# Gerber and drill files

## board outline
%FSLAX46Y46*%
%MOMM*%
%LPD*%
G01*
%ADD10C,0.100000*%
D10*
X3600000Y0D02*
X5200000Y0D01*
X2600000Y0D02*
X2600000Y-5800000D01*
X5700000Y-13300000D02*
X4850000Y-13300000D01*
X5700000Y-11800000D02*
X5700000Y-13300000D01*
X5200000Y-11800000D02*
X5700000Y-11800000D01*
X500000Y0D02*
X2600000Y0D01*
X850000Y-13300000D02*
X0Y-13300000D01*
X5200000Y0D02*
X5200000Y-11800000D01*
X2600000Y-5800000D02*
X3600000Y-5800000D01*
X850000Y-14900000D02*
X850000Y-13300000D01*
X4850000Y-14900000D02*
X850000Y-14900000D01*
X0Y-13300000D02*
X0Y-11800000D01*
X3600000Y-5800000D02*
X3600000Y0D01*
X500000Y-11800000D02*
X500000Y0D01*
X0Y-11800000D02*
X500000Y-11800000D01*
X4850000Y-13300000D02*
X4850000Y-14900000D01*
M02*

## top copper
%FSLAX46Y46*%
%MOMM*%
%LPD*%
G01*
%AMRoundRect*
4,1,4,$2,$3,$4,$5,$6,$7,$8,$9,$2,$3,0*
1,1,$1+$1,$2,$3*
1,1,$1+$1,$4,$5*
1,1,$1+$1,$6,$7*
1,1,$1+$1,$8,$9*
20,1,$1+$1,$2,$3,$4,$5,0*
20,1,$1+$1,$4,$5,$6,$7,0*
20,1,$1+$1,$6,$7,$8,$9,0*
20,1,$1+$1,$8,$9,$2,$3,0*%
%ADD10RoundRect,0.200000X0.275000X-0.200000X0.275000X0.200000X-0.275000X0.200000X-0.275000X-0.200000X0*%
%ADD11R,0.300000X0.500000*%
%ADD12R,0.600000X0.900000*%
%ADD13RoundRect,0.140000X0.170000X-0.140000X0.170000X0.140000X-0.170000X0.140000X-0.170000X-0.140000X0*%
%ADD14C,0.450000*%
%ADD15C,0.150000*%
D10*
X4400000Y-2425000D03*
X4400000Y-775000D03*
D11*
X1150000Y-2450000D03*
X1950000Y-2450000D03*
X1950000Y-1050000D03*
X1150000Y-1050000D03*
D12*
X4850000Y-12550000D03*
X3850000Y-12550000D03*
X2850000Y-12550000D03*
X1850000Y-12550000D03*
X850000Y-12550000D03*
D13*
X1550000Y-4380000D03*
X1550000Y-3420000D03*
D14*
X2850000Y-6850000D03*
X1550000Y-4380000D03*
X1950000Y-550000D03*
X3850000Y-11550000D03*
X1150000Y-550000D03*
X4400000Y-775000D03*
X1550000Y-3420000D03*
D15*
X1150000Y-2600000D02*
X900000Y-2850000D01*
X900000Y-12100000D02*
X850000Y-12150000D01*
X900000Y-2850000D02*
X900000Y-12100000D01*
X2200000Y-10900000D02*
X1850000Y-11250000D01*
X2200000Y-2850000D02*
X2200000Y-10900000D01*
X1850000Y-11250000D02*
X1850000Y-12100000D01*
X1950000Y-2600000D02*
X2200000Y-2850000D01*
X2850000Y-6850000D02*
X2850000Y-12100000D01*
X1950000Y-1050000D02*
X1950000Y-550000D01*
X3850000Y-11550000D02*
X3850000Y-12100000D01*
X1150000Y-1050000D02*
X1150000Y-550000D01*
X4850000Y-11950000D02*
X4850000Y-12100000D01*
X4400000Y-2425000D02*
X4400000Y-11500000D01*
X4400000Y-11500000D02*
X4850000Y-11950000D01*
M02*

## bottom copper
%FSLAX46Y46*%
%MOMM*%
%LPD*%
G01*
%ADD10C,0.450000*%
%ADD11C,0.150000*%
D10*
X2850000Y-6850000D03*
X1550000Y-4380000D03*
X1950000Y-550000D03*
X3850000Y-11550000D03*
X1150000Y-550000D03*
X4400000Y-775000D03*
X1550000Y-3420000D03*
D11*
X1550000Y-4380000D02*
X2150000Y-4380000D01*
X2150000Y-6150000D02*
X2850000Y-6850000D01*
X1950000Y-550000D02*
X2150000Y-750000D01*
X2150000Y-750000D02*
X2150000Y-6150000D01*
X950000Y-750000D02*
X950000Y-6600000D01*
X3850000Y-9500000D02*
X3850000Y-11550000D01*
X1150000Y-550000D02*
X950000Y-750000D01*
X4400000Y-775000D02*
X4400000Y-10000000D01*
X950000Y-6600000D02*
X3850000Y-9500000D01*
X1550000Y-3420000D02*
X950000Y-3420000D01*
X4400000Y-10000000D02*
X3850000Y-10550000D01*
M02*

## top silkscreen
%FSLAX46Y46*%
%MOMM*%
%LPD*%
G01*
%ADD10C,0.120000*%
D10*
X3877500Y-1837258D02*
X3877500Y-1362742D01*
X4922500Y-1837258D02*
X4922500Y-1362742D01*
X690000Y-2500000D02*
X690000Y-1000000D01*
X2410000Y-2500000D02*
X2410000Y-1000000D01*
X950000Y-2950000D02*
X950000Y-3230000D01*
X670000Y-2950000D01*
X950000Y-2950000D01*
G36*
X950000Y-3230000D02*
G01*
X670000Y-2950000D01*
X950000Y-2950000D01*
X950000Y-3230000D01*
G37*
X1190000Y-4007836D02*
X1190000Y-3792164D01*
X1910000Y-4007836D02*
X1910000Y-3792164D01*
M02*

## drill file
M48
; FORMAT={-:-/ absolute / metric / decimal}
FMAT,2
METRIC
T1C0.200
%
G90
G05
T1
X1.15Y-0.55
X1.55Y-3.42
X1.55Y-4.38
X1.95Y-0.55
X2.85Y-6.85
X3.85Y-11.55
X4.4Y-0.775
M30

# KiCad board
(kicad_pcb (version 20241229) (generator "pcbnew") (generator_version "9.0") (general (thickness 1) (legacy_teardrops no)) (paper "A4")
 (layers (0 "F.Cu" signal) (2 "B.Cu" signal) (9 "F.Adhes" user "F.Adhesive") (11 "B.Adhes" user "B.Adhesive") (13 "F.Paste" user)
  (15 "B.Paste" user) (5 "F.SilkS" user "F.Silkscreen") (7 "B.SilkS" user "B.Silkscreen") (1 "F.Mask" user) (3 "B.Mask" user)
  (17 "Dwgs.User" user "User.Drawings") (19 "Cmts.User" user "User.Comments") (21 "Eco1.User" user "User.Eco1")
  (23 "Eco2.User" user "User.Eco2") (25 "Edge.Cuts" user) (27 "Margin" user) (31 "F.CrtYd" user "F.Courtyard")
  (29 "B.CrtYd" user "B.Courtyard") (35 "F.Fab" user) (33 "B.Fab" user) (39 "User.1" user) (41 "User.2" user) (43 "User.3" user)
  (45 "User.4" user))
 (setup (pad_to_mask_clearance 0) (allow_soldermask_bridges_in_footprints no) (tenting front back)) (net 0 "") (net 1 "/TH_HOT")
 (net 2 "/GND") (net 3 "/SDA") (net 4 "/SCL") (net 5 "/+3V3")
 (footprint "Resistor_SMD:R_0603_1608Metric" (layer "F.Cu") (at 4.4 1.6 90)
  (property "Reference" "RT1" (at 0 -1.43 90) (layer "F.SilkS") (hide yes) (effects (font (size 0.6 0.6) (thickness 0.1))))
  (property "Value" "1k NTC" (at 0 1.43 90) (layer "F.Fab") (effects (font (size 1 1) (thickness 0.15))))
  (fp_line (start -0.237258 -0.5225) (end 0.237258 -0.5225) (stroke (width 0.12) (type solid)) (layer "F.SilkS"))
  (fp_line (start -0.237258 0.5225) (end 0.237258 0.5225) (stroke (width 0.12) (type solid)) (layer "F.SilkS"))
  (pad "1" smd roundrect (at -0.825 0 90) (size 0.8 0.95) (layers "F.Cu" "F.Mask" "F.Paste") (roundrect_rratio 0.25) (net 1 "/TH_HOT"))
  (pad "2" smd roundrect (at 0.825 0 90) (size 0.8 0.95) (layers "F.Cu" "F.Mask" "F.Paste") (roundrect_rratio 0.25) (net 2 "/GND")))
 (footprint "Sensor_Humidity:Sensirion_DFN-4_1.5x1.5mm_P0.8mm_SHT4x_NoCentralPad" (layer "F.Cu") (at 1.55 1.75 90)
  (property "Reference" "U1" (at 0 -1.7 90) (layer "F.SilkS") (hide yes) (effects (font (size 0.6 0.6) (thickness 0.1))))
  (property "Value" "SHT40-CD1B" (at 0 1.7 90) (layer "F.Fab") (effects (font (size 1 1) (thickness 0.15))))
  (fp_line (start -0.75 -0.86) (end 0.75 -0.86) (stroke (width 0.12) (type solid)) (layer "F.SilkS"))
  (fp_line (start -0.75 0.86) (end 0.75 0.86) (stroke (width 0.12) (type solid)) (layer "F.SilkS"))
  (fp_poly
   (pts (xy -1.2 -0.6) (xy -1.48 -0.6) (xy -1.2 -0.88) (xy -1.2 -0.6)) (stroke (width 0.12) (type solid)) (fill yes) (layer "F.SilkS"))
  (pad "1" smd rect (at -0.7 -0.4 90) (size 0.5 0.3) (layers "F.Cu" "F.Mask" "F.Paste") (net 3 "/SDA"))
  (pad "2" smd rect (at -0.7 0.4 90) (size 0.5 0.3) (layers "F.Cu" "F.Mask" "F.Paste") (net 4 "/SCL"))
  (pad "3" smd rect (at 0.7 0.4 90) (size 0.5 0.3) (layers "F.Cu" "F.Mask" "F.Paste") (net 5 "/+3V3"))
  (pad "4" smd rect (at 0.7 -0.4 90) (size 0.5 0.3) (layers "F.Cu" "F.Mask" "F.Paste") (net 2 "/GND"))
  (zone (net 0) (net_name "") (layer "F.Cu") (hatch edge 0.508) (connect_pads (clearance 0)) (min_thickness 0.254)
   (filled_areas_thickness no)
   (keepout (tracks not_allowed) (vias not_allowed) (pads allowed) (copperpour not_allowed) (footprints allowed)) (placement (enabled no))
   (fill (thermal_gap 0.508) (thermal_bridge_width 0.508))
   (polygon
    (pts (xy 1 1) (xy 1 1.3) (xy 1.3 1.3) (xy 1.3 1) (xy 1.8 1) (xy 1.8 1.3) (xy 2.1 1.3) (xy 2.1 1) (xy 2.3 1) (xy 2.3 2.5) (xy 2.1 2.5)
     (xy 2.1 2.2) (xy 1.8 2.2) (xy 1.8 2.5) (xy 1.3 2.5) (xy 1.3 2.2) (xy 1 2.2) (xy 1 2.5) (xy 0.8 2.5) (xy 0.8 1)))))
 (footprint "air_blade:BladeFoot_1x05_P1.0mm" (layer "F.Cu") (at 2.85 12.55)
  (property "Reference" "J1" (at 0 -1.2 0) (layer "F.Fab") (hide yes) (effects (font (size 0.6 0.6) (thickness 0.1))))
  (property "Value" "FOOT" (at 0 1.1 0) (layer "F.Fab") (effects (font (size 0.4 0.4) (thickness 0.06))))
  (pad "1" smd rect (at 2 0) (size 0.6 0.9) (layers "F.Cu" "F.Mask" "F.Paste") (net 1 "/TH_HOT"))
  (pad "2" smd rect (at 1 0) (size 0.6 0.9) (layers "F.Cu" "F.Mask" "F.Paste") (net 2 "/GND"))
  (pad "3" smd rect (at 0 0) (size 0.6 0.9) (layers "F.Cu" "F.Mask" "F.Paste") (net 5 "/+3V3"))
  (pad "4" smd rect (at -1 0) (size 0.6 0.9) (layers "F.Cu" "F.Mask" "F.Paste") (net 4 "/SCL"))
  (pad "5" smd rect (at -2 0) (size 0.6 0.9) (layers "F.Cu" "F.Mask" "F.Paste") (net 3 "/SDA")))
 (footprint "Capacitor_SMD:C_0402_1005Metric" (layer "F.Cu") (at 1.55 3.9 90)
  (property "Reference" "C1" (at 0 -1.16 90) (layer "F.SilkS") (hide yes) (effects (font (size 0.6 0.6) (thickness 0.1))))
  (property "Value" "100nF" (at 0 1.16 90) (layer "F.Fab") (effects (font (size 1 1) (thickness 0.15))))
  (fp_line (start -0.107836 -0.36) (end 0.107836 -0.36) (stroke (width 0.12) (type solid)) (layer "F.SilkS"))
  (fp_line (start -0.107836 0.36) (end 0.107836 0.36) (stroke (width 0.12) (type solid)) (layer "F.SilkS"))
  (pad "1" smd roundrect (at -0.48 0 90) (size 0.56 0.62) (layers "F.Cu" "F.Mask" "F.Paste") (roundrect_rratio 0.25) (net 5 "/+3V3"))
  (pad "2" smd roundrect (at 0.48 0 90) (size 0.56 0.62) (layers "F.Cu" "F.Mask" "F.Paste") (roundrect_rratio 0.25) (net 2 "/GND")))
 (gr_line (start 3.6 0) (end 5.2 0) (stroke (width 0.1) (type default)) (layer "Edge.Cuts"))
 (gr_line (start 2.6 0) (end 2.6 5.8) (stroke (width 0.1) (type default)) (layer "Edge.Cuts"))
 (gr_line (start 5.7 13.3) (end 4.85 13.3) (stroke (width 0.1) (type default)) (layer "Edge.Cuts"))
 (gr_line (start 5.7 11.8) (end 5.7 13.3) (stroke (width 0.1) (type default)) (layer "Edge.Cuts"))
 (gr_line (start 5.2 11.8) (end 5.7 11.8) (stroke (width 0.1) (type default)) (layer "Edge.Cuts"))
 (gr_line (start 0.5 0) (end 2.6 0) (stroke (width 0.1) (type default)) (layer "Edge.Cuts"))
 (gr_line (start 0.85 13.3) (end 0 13.3) (stroke (width 0.1) (type default)) (layer "Edge.Cuts"))
 (gr_line (start 5.2 0) (end 5.2 11.8) (stroke (width 0.1) (type default)) (layer "Edge.Cuts"))
 (gr_line (start 2.6 5.8) (end 3.6 5.8) (stroke (width 0.1) (type default)) (layer "Edge.Cuts"))
 (gr_line (start 0.85 14.9) (end 0.85 13.3) (stroke (width 0.1) (type default)) (layer "Edge.Cuts"))
 (gr_line (start 4.85 14.9) (end 0.85 14.9) (stroke (width 0.1) (type default)) (layer "Edge.Cuts"))
 (gr_line (start 0 13.3) (end 0 11.8) (stroke (width 0.1) (type default)) (layer "Edge.Cuts"))
 (gr_line (start 3.6 5.8) (end 3.6 0) (stroke (width 0.1) (type default)) (layer "Edge.Cuts"))
 (gr_line (start 0.5 11.8) (end 0.5 0) (stroke (width 0.1) (type default)) (layer "Edge.Cuts"))
 (gr_line (start 0 11.8) (end 0.5 11.8) (stroke (width 0.1) (type default)) (layer "Edge.Cuts"))
 (gr_line (start 4.85 13.3) (end 4.85 14.9) (stroke (width 0.1) (type default)) (layer "Edge.Cuts"))
 (segment (start 1.15 2.6) (end 0.9 2.85) (width 0.15) (locked yes) (layer "F.Cu") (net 3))
 (segment (start 0.9 12.1) (end 0.85 12.15) (width 0.15) (locked yes) (layer "F.Cu") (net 3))
 (segment (start 0.9 2.85) (end 0.9 12.1) (width 0.15) (locked yes) (layer "F.Cu") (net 3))
 (segment (start 2.2 10.9) (end 1.85 11.25) (width 0.15) (locked yes) (layer "F.Cu") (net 4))
 (segment (start 2.2 2.85) (end 2.2 10.9) (width 0.15) (locked yes) (layer "F.Cu") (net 4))
 (segment (start 1.85 11.25) (end 1.85 12.1) (width 0.15) (locked yes) (layer "F.Cu") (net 4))
 (segment (start 1.95 2.6) (end 2.2 2.85) (width 0.15) (locked yes) (layer "F.Cu") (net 4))
 (segment (start 2.85 6.85) (end 2.85 12.1) (width 0.15) (locked yes) (layer "F.Cu") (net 5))
 (segment (start 1.95 1.05) (end 1.95 0.55) (width 0.15) (locked yes) (layer "F.Cu") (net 5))
 (via (at 2.85 6.85) (size 0.45) (drill 0.2) (layers "F.Cu" "B.Cu") (locked yes) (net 5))
 (via (at 1.55 4.38) (size 0.45) (drill 0.2) (layers "F.Cu" "B.Cu") (locked yes) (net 5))
 (via (at 1.95 0.55) (size 0.45) (drill 0.2) (layers "F.Cu" "B.Cu") (locked yes) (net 5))
 (segment (start 1.55 4.38) (end 2.15 4.38) (width 0.15) (locked yes) (layer "B.Cu") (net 5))
 (segment (start 2.15 6.15) (end 2.85 6.85) (width 0.15) (locked yes) (layer "B.Cu") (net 5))
 (segment (start 1.95 0.55) (end 2.15 0.75) (width 0.15) (locked yes) (layer "B.Cu") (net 5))
 (segment (start 2.15 0.75) (end 2.15 6.15) (width 0.15) (locked yes) (layer "B.Cu") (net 5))
 (segment (start 3.85 11.55) (end 3.85 12.1) (width 0.15) (locked yes) (layer "F.Cu") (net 2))
 (segment (start 1.15 1.05) (end 1.15 0.55) (width 0.15) (locked yes) (layer "F.Cu") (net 2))
 (via (at 3.85 11.55) (size 0.45) (drill 0.2) (layers "F.Cu" "B.Cu") (locked yes) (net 2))
 (via (at 1.15 0.55) (size 0.45) (drill 0.2) (layers "F.Cu" "B.Cu") (locked yes) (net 2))
 (via (at 4.4 0.775) (size 0.45) (drill 0.2) (layers "F.Cu" "B.Cu") (locked yes) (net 2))
 (via (at 1.55 3.42) (size 0.45) (drill 0.2) (layers "F.Cu" "B.Cu") (locked yes) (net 2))
 (segment (start 0.95 0.75) (end 0.95 6.6) (width 0.15) (locked yes) (layer "B.Cu") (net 2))
 (segment (start 3.85 9.5) (end 3.85 11.55) (width 0.15) (locked yes) (layer "B.Cu") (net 2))
 (segment (start 1.15 0.55) (end 0.95 0.75) (width 0.15) (locked yes) (layer "B.Cu") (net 2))
 (segment (start 4.4 0.775) (end 4.4 10) (width 0.15) (locked yes) (layer "B.Cu") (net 2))
 (segment (start 0.95 6.6) (end 3.85 9.5) (width 0.15) (locked yes) (layer "B.Cu") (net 2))
 (segment (start 1.55 3.42) (end 0.95 3.42) (width 0.15) (locked yes) (layer "B.Cu") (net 2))
 (segment (start 4.4 10) (end 3.85 10.55) (width 0.15) (locked yes) (layer "B.Cu") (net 2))
 (segment (start 4.85 11.95) (end 4.85 12.1) (width 0.15) (locked yes) (layer "F.Cu") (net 1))
 (segment (start 4.4 2.425) (end 4.4 11.5) (width 0.15) (locked yes) (layer "F.Cu") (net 1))
 (segment (start 4.4 11.5) (end 4.85 11.95) (width 0.15) (locked yes) (layer "F.Cu") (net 1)))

